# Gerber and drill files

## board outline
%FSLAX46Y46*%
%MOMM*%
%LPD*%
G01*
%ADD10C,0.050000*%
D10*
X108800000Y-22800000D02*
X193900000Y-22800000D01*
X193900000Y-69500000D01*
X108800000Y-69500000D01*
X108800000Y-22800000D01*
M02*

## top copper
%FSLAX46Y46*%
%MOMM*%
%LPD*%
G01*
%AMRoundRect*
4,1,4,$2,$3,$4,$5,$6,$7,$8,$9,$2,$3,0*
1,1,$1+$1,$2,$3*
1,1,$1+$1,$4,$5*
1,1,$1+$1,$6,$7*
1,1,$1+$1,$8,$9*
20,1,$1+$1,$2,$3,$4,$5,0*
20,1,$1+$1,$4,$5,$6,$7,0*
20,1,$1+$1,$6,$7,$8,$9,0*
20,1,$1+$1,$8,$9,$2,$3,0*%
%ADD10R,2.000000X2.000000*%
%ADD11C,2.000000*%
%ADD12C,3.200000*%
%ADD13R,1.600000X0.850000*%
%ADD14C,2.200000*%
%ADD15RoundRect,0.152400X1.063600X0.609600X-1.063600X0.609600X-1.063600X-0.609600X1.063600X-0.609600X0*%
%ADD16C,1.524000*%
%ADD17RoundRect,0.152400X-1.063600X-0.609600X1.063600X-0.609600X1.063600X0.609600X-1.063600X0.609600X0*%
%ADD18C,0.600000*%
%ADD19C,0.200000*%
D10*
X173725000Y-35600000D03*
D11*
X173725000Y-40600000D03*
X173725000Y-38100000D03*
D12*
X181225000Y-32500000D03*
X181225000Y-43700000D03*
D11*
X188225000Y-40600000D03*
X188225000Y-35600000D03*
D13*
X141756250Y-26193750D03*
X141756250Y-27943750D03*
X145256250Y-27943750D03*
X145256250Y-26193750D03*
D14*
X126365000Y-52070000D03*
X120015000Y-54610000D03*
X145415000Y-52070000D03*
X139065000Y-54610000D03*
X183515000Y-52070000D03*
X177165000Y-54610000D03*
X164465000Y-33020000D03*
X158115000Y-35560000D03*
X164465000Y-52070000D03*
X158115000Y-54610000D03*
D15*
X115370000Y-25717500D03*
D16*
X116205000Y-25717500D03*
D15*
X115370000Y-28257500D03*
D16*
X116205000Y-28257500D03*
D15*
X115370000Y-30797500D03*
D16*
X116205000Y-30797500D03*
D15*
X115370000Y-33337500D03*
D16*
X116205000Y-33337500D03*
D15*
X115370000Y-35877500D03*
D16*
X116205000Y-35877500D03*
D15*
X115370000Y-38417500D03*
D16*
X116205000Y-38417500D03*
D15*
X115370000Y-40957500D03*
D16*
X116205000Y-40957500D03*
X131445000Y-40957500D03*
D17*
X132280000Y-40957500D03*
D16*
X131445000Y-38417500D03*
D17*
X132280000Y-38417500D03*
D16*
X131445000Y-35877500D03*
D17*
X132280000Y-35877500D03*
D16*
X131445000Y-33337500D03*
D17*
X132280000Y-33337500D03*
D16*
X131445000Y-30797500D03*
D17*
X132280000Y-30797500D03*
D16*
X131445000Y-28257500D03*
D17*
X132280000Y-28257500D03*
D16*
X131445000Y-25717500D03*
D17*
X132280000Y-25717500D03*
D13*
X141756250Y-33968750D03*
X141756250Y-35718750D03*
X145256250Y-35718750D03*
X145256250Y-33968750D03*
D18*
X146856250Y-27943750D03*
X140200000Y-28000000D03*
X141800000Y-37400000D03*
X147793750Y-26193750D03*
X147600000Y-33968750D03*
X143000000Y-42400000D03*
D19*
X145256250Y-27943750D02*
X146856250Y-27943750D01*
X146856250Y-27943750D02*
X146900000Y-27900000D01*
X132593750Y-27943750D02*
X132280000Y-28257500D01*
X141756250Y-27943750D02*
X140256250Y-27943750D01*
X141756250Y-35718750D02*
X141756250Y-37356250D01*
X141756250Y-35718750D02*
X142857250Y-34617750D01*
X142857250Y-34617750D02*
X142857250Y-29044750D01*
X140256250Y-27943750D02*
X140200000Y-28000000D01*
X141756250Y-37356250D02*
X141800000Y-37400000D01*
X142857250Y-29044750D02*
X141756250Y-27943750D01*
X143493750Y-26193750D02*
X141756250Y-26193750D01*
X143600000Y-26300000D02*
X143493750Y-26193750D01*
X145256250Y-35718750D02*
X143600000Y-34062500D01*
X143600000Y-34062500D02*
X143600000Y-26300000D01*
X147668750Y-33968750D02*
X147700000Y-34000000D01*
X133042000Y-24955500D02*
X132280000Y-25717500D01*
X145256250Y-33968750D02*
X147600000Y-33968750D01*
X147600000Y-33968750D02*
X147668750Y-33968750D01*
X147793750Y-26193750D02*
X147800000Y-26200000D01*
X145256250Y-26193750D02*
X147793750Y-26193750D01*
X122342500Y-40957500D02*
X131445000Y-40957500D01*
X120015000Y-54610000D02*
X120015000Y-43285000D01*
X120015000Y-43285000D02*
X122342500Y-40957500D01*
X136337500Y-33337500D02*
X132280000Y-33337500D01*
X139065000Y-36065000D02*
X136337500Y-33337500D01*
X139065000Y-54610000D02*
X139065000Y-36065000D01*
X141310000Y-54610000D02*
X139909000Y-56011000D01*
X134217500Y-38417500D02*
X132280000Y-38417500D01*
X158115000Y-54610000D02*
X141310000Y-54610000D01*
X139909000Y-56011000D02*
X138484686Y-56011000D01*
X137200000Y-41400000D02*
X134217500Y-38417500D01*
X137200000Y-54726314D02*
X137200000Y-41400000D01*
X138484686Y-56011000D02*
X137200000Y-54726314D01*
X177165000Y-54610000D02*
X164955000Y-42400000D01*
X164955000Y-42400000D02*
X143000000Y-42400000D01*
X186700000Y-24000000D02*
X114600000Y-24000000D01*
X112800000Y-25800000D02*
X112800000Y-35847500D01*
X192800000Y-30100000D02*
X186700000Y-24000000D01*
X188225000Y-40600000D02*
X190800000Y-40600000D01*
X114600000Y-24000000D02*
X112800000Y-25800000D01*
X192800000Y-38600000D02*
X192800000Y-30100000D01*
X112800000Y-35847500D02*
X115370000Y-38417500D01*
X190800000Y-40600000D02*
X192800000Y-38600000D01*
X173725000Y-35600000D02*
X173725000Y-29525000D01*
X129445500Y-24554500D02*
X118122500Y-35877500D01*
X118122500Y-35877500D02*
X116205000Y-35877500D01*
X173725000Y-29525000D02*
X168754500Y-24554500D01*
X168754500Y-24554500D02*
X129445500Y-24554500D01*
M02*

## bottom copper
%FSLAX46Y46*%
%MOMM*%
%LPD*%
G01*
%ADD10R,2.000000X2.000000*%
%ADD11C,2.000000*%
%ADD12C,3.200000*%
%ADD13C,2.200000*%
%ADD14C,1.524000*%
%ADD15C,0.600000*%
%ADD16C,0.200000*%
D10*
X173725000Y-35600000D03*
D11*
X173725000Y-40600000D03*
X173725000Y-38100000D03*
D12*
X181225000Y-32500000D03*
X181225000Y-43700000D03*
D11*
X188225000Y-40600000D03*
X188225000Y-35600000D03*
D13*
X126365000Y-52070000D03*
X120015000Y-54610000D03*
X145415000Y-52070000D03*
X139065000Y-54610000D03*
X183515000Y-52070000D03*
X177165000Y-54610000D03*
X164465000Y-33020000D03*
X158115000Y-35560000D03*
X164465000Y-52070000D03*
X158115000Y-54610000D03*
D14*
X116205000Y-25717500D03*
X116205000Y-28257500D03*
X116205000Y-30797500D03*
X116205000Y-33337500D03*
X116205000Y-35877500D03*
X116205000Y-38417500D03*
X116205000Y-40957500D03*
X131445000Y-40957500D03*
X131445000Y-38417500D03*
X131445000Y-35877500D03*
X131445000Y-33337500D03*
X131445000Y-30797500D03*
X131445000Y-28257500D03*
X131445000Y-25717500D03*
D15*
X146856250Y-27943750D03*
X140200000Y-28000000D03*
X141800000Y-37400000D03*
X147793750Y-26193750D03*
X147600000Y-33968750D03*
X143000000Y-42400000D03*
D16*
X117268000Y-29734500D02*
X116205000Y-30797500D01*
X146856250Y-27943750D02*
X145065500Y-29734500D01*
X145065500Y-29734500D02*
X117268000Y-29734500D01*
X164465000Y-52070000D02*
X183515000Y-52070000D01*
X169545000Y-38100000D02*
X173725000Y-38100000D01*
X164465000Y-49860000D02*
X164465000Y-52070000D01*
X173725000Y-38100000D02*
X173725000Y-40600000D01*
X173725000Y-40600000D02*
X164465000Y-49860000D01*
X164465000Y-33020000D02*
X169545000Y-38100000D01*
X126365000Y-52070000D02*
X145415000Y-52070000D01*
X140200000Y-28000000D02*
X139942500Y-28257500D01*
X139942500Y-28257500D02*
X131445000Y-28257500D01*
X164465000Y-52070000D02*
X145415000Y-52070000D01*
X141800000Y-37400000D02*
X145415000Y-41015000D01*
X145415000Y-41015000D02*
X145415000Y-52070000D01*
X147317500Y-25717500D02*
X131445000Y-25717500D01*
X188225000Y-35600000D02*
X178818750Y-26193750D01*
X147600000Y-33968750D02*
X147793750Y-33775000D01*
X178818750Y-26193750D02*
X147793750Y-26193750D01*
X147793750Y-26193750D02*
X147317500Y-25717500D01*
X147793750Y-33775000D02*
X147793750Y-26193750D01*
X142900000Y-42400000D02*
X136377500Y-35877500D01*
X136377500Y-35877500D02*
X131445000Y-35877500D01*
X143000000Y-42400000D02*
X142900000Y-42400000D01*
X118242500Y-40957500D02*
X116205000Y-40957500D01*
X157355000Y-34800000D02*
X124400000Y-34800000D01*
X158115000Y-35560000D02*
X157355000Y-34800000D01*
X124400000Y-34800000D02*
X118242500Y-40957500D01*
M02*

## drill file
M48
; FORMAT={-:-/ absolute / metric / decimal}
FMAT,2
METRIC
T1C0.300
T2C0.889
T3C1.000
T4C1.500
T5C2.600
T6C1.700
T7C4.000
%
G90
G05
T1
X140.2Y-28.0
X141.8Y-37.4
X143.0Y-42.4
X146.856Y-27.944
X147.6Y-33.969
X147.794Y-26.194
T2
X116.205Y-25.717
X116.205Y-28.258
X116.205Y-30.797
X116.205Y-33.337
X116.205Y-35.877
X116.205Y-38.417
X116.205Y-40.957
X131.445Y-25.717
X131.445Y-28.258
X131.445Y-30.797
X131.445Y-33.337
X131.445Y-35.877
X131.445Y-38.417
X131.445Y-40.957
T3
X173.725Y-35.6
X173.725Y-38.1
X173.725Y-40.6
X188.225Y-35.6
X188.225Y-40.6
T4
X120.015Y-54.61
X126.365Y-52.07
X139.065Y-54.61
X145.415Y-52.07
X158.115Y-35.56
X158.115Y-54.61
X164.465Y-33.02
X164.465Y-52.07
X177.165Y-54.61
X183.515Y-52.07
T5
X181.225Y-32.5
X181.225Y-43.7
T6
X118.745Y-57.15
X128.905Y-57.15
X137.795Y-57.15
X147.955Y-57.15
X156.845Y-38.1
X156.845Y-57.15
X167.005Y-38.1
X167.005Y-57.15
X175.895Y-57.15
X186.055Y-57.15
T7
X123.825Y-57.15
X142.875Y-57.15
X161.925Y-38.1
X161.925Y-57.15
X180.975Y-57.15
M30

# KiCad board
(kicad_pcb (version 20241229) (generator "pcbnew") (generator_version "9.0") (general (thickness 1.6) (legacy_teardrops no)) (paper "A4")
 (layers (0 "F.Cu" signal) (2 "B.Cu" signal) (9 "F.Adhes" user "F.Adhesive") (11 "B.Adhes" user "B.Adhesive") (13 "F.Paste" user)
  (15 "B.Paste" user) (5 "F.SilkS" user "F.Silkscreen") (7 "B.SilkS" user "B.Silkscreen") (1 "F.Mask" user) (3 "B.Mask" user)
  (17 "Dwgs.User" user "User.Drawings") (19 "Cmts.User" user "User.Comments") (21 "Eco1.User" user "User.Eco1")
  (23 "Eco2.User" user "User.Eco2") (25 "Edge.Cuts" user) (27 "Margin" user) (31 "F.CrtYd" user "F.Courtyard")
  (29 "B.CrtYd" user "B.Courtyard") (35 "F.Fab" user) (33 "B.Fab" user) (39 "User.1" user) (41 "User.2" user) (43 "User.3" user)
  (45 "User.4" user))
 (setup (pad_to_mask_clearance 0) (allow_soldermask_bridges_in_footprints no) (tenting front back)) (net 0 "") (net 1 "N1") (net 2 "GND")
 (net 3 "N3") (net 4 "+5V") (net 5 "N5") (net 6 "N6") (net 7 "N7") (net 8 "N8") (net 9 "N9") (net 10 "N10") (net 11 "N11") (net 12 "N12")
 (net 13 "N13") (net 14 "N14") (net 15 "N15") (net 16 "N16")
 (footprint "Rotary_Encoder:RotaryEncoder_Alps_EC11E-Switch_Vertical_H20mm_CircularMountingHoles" (layer "F.Cu") (at 173.725 35.6)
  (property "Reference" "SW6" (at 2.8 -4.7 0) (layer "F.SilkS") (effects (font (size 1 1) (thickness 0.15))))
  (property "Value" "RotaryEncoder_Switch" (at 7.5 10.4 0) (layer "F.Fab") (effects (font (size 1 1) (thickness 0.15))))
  (pad "A" thru_hole rect (at 0 0) (size 2 2) (drill 1) (layers "*.Cu" "*.Mask") (remove_unused_layers no) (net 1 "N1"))
  (pad "B" thru_hole circle (at 0 5) (size 2 2) (drill 1) (layers "*.Cu" "*.Mask") (remove_unused_layers no) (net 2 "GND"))
  (pad "C" thru_hole circle (at 0 2.5) (size 2 2) (drill 1) (layers "*.Cu" "*.Mask") (remove_unused_layers no) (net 2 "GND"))
  (pad "MP" thru_hole circle (at 7.5 -3.1) (size 3.2 3.2) (drill 2.6) (layers "*.Cu" "*.Mask") (remove_unused_layers no))
  (pad "MP" thru_hole circle (at 7.5 8.1) (size 3.2 3.2) (drill 2.6) (layers "*.Cu" "*.Mask") (remove_unused_layers no))
  (pad "S1" thru_hole circle (at 14.5 5) (size 2 2) (drill 1) (layers "*.Cu" "*.Mask") (remove_unused_layers no) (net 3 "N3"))
  (pad "S2" thru_hole circle (at 14.5 0) (size 2 2) (drill 1) (layers "*.Cu" "*.Mask") (remove_unused_layers no) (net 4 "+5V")))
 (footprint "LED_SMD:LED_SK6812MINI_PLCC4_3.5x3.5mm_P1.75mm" (layer "F.Cu") (at 143.50625 27.06875)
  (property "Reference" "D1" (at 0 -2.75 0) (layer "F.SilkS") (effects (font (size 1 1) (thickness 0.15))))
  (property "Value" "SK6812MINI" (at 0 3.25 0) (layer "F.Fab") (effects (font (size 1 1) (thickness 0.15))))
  (pad "1" smd rect (at -1.75 -0.875) (size 1.6 0.85) (layers "F.Cu" "F.Mask" "F.Paste") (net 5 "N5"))
  (pad "2" smd rect (at -1.75 0.875) (size 1.6 0.85) (layers "F.Cu" "F.Mask" "F.Paste") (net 2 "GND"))
  (pad "3" smd rect (at 1.75 0.875) (size 1.6 0.85) (layers "F.Cu" "F.Mask" "F.Paste") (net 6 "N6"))
  (pad "4" smd rect (at 1.75 -0.875) (size 1.6 0.85) (layers "F.Cu" "F.Mask" "F.Paste") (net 4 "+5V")))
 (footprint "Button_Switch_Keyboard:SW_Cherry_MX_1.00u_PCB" (layer "F.Cu") (at 126.365 52.07)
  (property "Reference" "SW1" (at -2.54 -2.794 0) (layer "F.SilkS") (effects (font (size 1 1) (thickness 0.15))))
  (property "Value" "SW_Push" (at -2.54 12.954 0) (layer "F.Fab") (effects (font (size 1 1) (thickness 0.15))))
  (pad "" np_thru_hole circle (at -7.62 5.08) (size 1.7 1.7) (drill 1.7) (layers "*.Cu" "*.Mask"))
  (pad "" np_thru_hole circle (at -2.54 5.08) (size 4 4) (drill 4) (layers "*.Cu" "*.Mask"))
  (pad "" np_thru_hole circle (at 2.54 5.08) (size 1.7 1.7) (drill 1.7) (layers "*.Cu" "*.Mask"))
  (pad "1" thru_hole circle (at 0 0) (size 2.2 2.2) (drill 1.5) (layers "*.Cu" "*.Mask") (remove_unused_layers no) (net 2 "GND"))
  (pad "2" thru_hole circle (at -6.35 2.54) (size 2.2 2.2) (drill 1.5) (layers "*.Cu" "*.Mask") (remove_unused_layers no) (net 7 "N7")))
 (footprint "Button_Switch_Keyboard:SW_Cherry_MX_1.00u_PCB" (layer "F.Cu") (at 145.415 52.07)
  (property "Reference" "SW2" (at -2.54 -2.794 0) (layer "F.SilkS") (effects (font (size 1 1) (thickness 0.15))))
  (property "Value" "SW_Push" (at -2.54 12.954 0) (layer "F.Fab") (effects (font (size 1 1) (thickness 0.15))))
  (pad "" np_thru_hole circle (at -7.62 5.08) (size 1.7 1.7) (drill 1.7) (layers "*.Cu" "*.Mask"))
  (pad "" np_thru_hole circle (at -2.54 5.08) (size 4 4) (drill 4) (layers "*.Cu" "*.Mask"))
  (pad "" np_thru_hole circle (at 2.54 5.08) (size 1.7 1.7) (drill 1.7) (layers "*.Cu" "*.Mask"))
  (pad "1" thru_hole circle (at 0 0) (size 2.2 2.2) (drill 1.5) (layers "*.Cu" "*.Mask") (remove_unused_layers no) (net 2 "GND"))
  (pad "2" thru_hole circle (at -6.35 2.54) (size 2.2 2.2) (drill 1.5) (layers "*.Cu" "*.Mask") (remove_unused_layers no) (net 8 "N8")))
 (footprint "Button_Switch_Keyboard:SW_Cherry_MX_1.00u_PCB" (layer "F.Cu") (at 183.515 52.07)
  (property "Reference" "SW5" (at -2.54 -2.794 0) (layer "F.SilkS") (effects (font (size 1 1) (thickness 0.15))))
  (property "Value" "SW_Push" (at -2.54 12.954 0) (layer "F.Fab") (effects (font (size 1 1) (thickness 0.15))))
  (pad "" np_thru_hole circle (at -7.62 5.08) (size 1.7 1.7) (drill 1.7) (layers "*.Cu" "*.Mask"))
  (pad "" np_thru_hole circle (at -2.54 5.08) (size 4 4) (drill 4) (layers "*.Cu" "*.Mask"))
  (pad "" np_thru_hole circle (at 2.54 5.08) (size 1.7 1.7) (drill 1.7) (layers "*.Cu" "*.Mask"))
  (pad "1" thru_hole circle (at 0 0) (size 2.2 2.2) (drill 1.5) (layers "*.Cu" "*.Mask") (remove_unused_layers no) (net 2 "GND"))
  (pad "2" thru_hole circle (at -6.35 2.54) (size 2.2 2.2) (drill 1.5) (layers "*.Cu" "*.Mask") (remove_unused_layers no) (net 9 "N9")))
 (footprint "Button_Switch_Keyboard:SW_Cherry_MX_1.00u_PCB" (layer "F.Cu") (at 164.465 33.02)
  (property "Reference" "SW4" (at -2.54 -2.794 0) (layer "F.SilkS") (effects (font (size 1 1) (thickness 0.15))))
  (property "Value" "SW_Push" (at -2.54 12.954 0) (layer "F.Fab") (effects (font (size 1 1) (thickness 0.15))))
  (pad "" np_thru_hole circle (at -7.62 5.08) (size 1.7 1.7) (drill 1.7) (layers "*.Cu" "*.Mask"))
  (pad "" np_thru_hole circle (at -2.54 5.08) (size 4 4) (drill 4) (layers "*.Cu" "*.Mask"))
  (pad "" np_thru_hole circle (at 2.54 5.08) (size 1.7 1.7) (drill 1.7) (layers "*.Cu" "*.Mask"))
  (pad "1" thru_hole circle (at 0 0) (size 2.2 2.2) (drill 1.5) (layers "*.Cu" "*.Mask") (remove_unused_layers no) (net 2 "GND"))
  (pad "2" thru_hole circle (at -6.35 2.54) (size 2.2 2.2) (drill 1.5) (layers "*.Cu" "*.Mask") (remove_unused_layers no) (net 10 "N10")))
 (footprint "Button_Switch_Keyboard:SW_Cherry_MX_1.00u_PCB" (layer "F.Cu") (at 164.465 52.07)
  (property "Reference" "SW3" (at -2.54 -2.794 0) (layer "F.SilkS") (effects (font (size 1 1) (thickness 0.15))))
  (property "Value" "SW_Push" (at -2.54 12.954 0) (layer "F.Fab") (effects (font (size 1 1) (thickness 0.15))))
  (pad "" np_thru_hole circle (at -7.62 5.08) (size 1.7 1.7) (drill 1.7) (layers "*.Cu" "*.Mask"))
  (pad "" np_thru_hole circle (at -2.54 5.08) (size 4 4) (drill 4) (layers "*.Cu" "*.Mask"))
  (pad "" np_thru_hole circle (at 2.54 5.08) (size 1.7 1.7) (drill 1.7) (layers "*.Cu" "*.Mask"))
  (pad "1" thru_hole circle (at 0 0) (size 2.2 2.2) (drill 1.5) (layers "*.Cu" "*.Mask") (remove_unused_layers no) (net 2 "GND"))
  (pad "2" thru_hole circle (at -6.35 2.54) (size 2.2 2.2) (drill 1.5) (layers "*.Cu" "*.Mask") (remove_unused_layers no) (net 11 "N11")))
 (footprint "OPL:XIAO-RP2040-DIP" (layer "F.Cu") (at 123.825 33.3375)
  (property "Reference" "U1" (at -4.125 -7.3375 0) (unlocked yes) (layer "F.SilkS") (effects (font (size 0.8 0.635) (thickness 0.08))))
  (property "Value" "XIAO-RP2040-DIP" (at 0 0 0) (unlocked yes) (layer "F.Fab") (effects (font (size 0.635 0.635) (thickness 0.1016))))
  (pad "1" smd roundrect (at -8.455 -7.62 180) (size 2.432 1.524) (layers "F.Cu" "F.Mask") (roundrect_rratio 0.1) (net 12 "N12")
   (thermal_bridge_angle 45))
  (pad "1" thru_hole circle (at -7.62 -7.62 180) (size 1.524 1.524) (drill 0.889) (layers "*.Cu" "*.Mask") (remove_unused_layers no)
   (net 12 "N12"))
  (pad "2" smd roundrect (at -8.455 -5.08 180) (size 2.432 1.524) (layers "F.Cu" "F.Mask") (roundrect_rratio 0.1) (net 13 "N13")
   (thermal_bridge_angle 45))
  (pad "2" thru_hole circle (at -7.62 -5.08 180) (size 1.524 1.524) (drill 0.889) (layers "*.Cu" "*.Mask") (remove_unused_layers no)
   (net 13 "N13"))
  (pad "3" smd roundrect (at -8.455 -2.54 180) (size 2.432 1.524) (layers "F.Cu" "F.Mask") (roundrect_rratio 0.1) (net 6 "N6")
   (thermal_bridge_angle 45))
  (pad "3" thru_hole circle (at -7.62 -2.54 180) (size 1.524 1.524) (drill 0.889) (layers "*.Cu" "*.Mask") (remove_unused_layers no)
   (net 6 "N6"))
  (pad "4" smd roundrect (at -8.455 0 180) (size 2.432 1.524) (layers "F.Cu" "F.Mask") (roundrect_rratio 0.1) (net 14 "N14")
   (thermal_bridge_angle 45))
  (pad "4" thru_hole circle (at -7.62 0 180) (size 1.524 1.524) (drill 0.889) (layers "*.Cu" "*.Mask") (remove_unused_layers no)
   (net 14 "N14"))
  (pad "5" smd roundrect (at -8.455 2.54 180) (size 2.432 1.524) (layers "F.Cu" "F.Mask") (roundrect_rratio 0.1) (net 1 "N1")
   (thermal_bridge_angle 45))
  (pad "5" thru_hole circle (at -7.62 2.54 180) (size 1.524 1.524) (drill 0.889) (layers "*.Cu" "*.Mask") (remove_unused_layers no)
   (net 1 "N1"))
  (pad "6" smd roundrect (at -8.455 5.08 180) (size 2.432 1.524) (layers "F.Cu" "F.Mask") (roundrect_rratio 0.1) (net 3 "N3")
   (thermal_bridge_angle 45))
  (pad "6" thru_hole circle (at -7.62 5.08 180) (size 1.524 1.524) (drill 0.889) (layers "*.Cu" "*.Mask") (remove_unused_layers no)
   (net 3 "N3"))
  (pad "7" smd roundrect (at -8.455 7.62 180) (size 2.432 1.524) (layers "F.Cu" "F.Mask") (roundrect_rratio 0.1) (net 10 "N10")
   (thermal_bridge_angle 45))
  (pad "7" thru_hole circle (at -7.62 7.62 180) (size 1.524 1.524) (drill 0.889) (layers "*.Cu" "*.Mask") (remove_unused_layers no)
   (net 10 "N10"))
  (pad "8" thru_hole circle (at 7.62 7.62) (size 1.524 1.524) (drill 0.889) (layers "*.Cu" "*.Mask") (remove_unused_layers no) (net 7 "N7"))
  (pad "8" smd roundrect (at 8.455 7.62) (size 2.432 1.524) (layers "F.Cu" "F.Mask") (roundrect_rratio 0.1) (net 7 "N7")
   (thermal_bridge_angle 45))
  (pad "9" thru_hole circle (at 7.62 5.08) (size 1.524 1.524) (drill 0.889) (layers "*.Cu" "*.Mask") (remove_unused_layers no)
   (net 11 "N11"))
  (pad "9" smd roundrect (at 8.455 5.08) (size 2.432 1.524) (layers "F.Cu" "F.Mask") (roundrect_rratio 0.1) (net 11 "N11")
   (thermal_bridge_angle 45))
  (pad "10" thru_hole circle (at 7.62 2.54) (size 1.524 1.524) (drill 0.889) (layers "*.Cu" "*.Mask") (remove_unused_layers no) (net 9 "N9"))
  (pad "10" smd roundrect (at 8.455 2.54) (size 2.432 1.524) (layers "F.Cu" "F.Mask") (roundrect_rratio 0.1) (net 9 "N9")
   (thermal_bridge_angle 45))
  (pad "11" thru_hole circle (at 7.62 0) (size 1.524 1.524) (drill 0.889) (layers "*.Cu" "*.Mask") (remove_unused_layers no) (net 8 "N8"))
  (pad "11" smd roundrect (at 8.455 0) (size 2.432 1.524) (layers "F.Cu" "F.Mask") (roundrect_rratio 0.1) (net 8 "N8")
   (thermal_bridge_angle 45))
  (pad "12" thru_hole circle (at 7.62 -2.54) (size 1.524 1.524) (drill 0.889) (layers "*.Cu" "*.Mask") (remove_unused_layers no)
   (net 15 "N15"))
  (pad "12" smd roundrect (at 8.455 -2.54) (size 2.432 1.524) (layers "F.Cu" "F.Mask") (roundrect_rratio 0.1) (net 15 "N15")
   (thermal_bridge_angle 45))
  (pad "13" thru_hole circle (at 7.62 -5.08) (size 1.524 1.524) (drill 0.889) (layers "*.Cu" "*.Mask") (remove_unused_layers no)
   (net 2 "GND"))
  (pad "13" smd roundrect (at 8.455 -5.08) (size 2.432 1.524) (layers "F.Cu" "F.Mask") (roundrect_rratio 0.1) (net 2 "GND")
   (thermal_bridge_angle 45))
  (pad "14" thru_hole circle (at 7.62 -7.62) (size 1.524 1.524) (drill 0.889) (layers "*.Cu" "*.Mask") (remove_unused_layers no)
   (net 4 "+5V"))
  (pad "14" smd roundrect (at 8.455 -7.62) (size 2.432 1.524) (layers "F.Cu" "F.Mask") (roundrect_rratio 0.1) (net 4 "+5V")
   (thermal_bridge_angle 45)))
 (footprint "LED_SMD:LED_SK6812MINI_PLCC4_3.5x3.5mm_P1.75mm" (layer "F.Cu") (at 143.50625 34.84375)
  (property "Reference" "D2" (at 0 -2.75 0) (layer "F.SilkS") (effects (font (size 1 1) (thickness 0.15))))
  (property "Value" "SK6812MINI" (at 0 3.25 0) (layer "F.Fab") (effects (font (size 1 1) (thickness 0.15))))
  (pad "1" smd rect (at -1.75 -0.875) (size 1.6 0.85) (layers "F.Cu" "F.Mask" "F.Paste") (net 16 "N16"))
  (pad "2" smd rect (at -1.75 0.875) (size 1.6 0.85) (layers "F.Cu" "F.Mask" "F.Paste") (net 2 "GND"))
  (pad "3" smd rect (at 1.75 0.875) (size 1.6 0.85) (layers "F.Cu" "F.Mask" "F.Paste") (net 5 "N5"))
  (pad "4" smd rect (at 1.75 -0.875) (size 1.6 0.85) (layers "F.Cu" "F.Mask" "F.Paste") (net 4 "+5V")))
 (gr_rect (start 108.8 22.8) (end 193.9 69.5) (stroke (width 0.05) (type default)) (fill no) (layer "Edge.Cuts"))
 (segment (start 145.25625 27.94375) (end 146.85625 27.94375) (width 0.2) (layer "F.Cu") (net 6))
 (segment (start 146.85625 27.94375) (end 146.9 27.9) (width 0.2) (layer "F.Cu") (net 6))
 (via (at 146.85625 27.94375) (size 0.6) (drill 0.3) (layers "F.Cu" "B.Cu") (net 6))
 (segment (start 117.268 29.7345) (end 116.205 30.7975) (width 0.2) (layer "B.Cu") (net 6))
 (segment (start 146.85625 27.94375) (end 145.0655 29.7345) (width 0.2) (layer "B.Cu") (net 6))
 (segment (start 145.0655 29.7345) (end 117.268 29.7345) (width 0.2) (layer "B.Cu") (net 6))
 (segment (start 132.59375 27.94375) (end 132.28 28.2575) (width 0.2) (layer "F.Cu") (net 2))
 (segment (start 141.75625 27.94375) (end 140.25625 27.94375) (width 0.2) (layer "F.Cu") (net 2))
 (segment (start 141.75625 35.71875) (end 141.75625 37.35625) (width 0.2) (layer "F.Cu") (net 2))
 (segment (start 141.75625 35.71875) (end 142.85725 34.61775) (width 0.2) (layer "F.Cu") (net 2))
 (segment (start 142.85725 34.61775) (end 142.85725 29.04475) (width 0.2) (layer "F.Cu") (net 2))
 (segment (start 140.25625 27.94375) (end 140.2 28) (width 0.2) (layer "F.Cu") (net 2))
 (segment (start 141.75625 37.35625) (end 141.8 37.4) (width 0.2) (layer "F.Cu") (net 2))
 (segment (start 142.85725 29.04475) (end 141.75625 27.94375) (width 0.2) (layer "F.Cu") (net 2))
 (via (at 140.2 28) (size 0.6) (drill 0.3) (layers "F.Cu" "B.Cu") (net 2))
 (via (at 141.8 37.4) (size 0.6) (drill 0.3) (layers "F.Cu" "B.Cu") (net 2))
 (segment (start 164.465 52.07) (end 183.515 52.07) (width 0.2) (layer "B.Cu") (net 2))
 (segment (start 169.545 38.1) (end 173.725 38.1) (width 0.2) (layer "B.Cu") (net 2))
 (segment (start 164.465 49.86) (end 164.465 52.07) (width 0.2) (layer "B.Cu") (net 2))
 (segment (start 173.725 38.1) (end 173.725 40.6) (width 0.2) (layer "B.Cu") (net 2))
 (segment (start 173.725 40.6) (end 164.465 49.86) (width 0.2) (layer "B.Cu") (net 2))
 (segment (start 164.465 33.02) (end 169.545 38.1) (width 0.2) (layer "B.Cu") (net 2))
 (segment (start 126.365 52.07) (end 145.415 52.07) (width 0.2) (layer "B.Cu") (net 2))
 (segment (start 140.2 28) (end 139.9425 28.2575) (width 0.2) (layer "B.Cu") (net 2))
 (segment (start 139.9425 28.2575) (end 131.445 28.2575) (width 0.2) (layer "B.Cu") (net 2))
 (segment (start 164.465 52.07) (end 145.415 52.07) (width 0.2) (layer "B.Cu") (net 2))
 (segment (start 141.8 37.4) (end 145.415 41.015) (width 0.2) (layer "B.Cu") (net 2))
 (segment (start 145.415 41.015) (end 145.415 52.07) (width 0.2) (layer "B.Cu") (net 2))
 (segment (start 143.49375 26.19375) (end 141.75625 26.19375) (width 0.2) (layer "F.Cu") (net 5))
 (segment (start 143.6 26.3) (end 143.49375 26.19375) (width 0.2) (layer "F.Cu") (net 5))
 (segment (start 145.25625 35.71875) (end 143.6 34.0625) (width 0.2) (layer "F.Cu") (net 5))
 (segment (start 143.6 34.0625) (end 143.6 26.3) (width 0.2) (layer "F.Cu") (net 5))
 (segment (start 147.66875 33.96875) (end 147.7 34) (width 0.2) (layer "F.Cu") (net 4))
 (segment (start 133.042 24.9555) (end 132.28 25.7175) (width 0.2) (layer "F.Cu") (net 4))
 (segment (start 145.25625 33.96875) (end 147.6 33.96875) (width 0.2) (layer "F.Cu") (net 4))
 (segment (start 147.6 33.96875) (end 147.66875 33.96875) (width 0.2) (layer "F.Cu") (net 4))
 (segment (start 147.79375 26.19375) (end 147.8 26.2) (width 0.2) (layer "F.Cu") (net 4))
 (segment (start 145.25625 26.19375) (end 147.79375 26.19375) (width 0.2) (layer "F.Cu") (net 4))
 (via (at 147.79375 26.19375) (size 0.6) (drill 0.3) (layers "F.Cu" "B.Cu") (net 4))
 (via (at 147.6 33.96875) (size 0.6) (drill 0.3) (layers "F.Cu" "B.Cu") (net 4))
 (segment (start 147.3175 25.7175) (end 131.445 25.7175) (width 0.2) (layer "B.Cu") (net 4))
 (segment (start 188.225 35.6) (end 178.81875 26.19375) (width 0.2) (layer "B.Cu") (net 4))
 (segment (start 147.6 33.96875) (end 147.79375 33.775) (width 0.2) (layer "B.Cu") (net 4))
 (segment (start 178.81875 26.19375) (end 147.79375 26.19375) (width 0.2) (layer "B.Cu") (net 4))
 (segment (start 147.79375 26.19375) (end 147.3175 25.7175) (width 0.2) (layer "B.Cu") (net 4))
 (segment (start 147.79375 33.775) (end 147.79375 26.19375) (width 0.2) (layer "B.Cu") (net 4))
 (segment (start 122.3425 40.9575) (end 131.445 40.9575) (width 0.2) (layer "F.Cu") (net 7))
 (segment (start 120.015 54.61) (end 120.015 43.285) (width 0.2) (layer "F.Cu") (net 7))
 (segment (start 120.015 43.285) (end 122.3425 40.9575) (width 0.2) (layer "F.Cu") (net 7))
 (segment (start 136.3375 33.3375) (end 132.28 33.3375) (width 0.2) (layer "F.Cu") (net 8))
 (segment (start 139.065 36.065) (end 136.3375 33.3375) (width 0.2) (layer "F.Cu") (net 8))
 (segment (start 139.065 54.61) (end 139.065 36.065) (width 0.2) (layer "F.Cu") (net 8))
 (segment (start 141.31 54.61) (end 139.909 56.011) (width 0.2) (layer "F.Cu") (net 11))
 (segment (start 134.2175 38.4175) (end 132.28 38.4175) (width 0.2) (layer "F.Cu") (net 11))
 (segment (start 158.115 54.61) (end 141.31 54.61) (width 0.2) (layer "F.Cu") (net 11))
 (segment (start 139.909 56.011) (end 138.484686 56.011) (width 0.2) (layer "F.Cu") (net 11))
 (segment (start 137.2 41.4) (end 134.2175 38.4175) (width 0.2) (layer "F.Cu") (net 11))
 (segment (start 137.2 54.726314) (end 137.2 41.4) (width 0.2) (layer "F.Cu") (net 11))
 (segment (start 138.484686 56.011) (end 137.2 54.726314) (width 0.2) (layer "F.Cu") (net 11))
 (segment (start 177.165 54.61) (end 164.955 42.4) (width 0.2) (layer "F.Cu") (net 9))
 (segment (start 164.955 42.4) (end 143 42.4) (width 0.2) (layer "F.Cu") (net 9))
 (via (at 143 42.4) (size 0.6) (drill 0.3) (layers "F.Cu" "B.Cu") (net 9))
 (segment (start 142.9 42.4) (end 136.3775 35.8775) (width 0.2) (layer "B.Cu") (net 9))
 (segment (start 136.3775 35.8775) (end 131.445 35.8775) (width 0.2) (layer "B.Cu") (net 9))
 (segment (start 143 42.4) (end 142.9 42.4) (width 0.2) (layer "B.Cu") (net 9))
 (segment (start 118.2425 40.9575) (end 116.205 40.9575) (width 0.2) (layer "B.Cu") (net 10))
 (segment (start 157.355 34.8) (end 124.4 34.8) (width 0.2) (layer "B.Cu") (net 10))
 (segment (start 158.115 35.56) (end 157.355 34.8) (width 0.2) (layer "B.Cu") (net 10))
 (segment (start 124.4 34.8) (end 118.2425 40.9575) (width 0.2) (layer "B.Cu") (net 10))
 (segment (start 186.7 24) (end 114.6 24) (width 0.2) (layer "F.Cu") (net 3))
 (segment (start 112.8 25.8) (end 112.8 35.8475) (width 0.2) (layer "F.Cu") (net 3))
 (segment (start 192.8 30.1) (end 186.7 24) (width 0.2) (layer "F.Cu") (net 3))
 (segment (start 188.225 40.6) (end 190.8 40.6) (width 0.2) (layer "F.Cu") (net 3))
 (segment (start 114.6 24) (end 112.8 25.8) (width 0.2) (layer "F.Cu") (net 3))
 (segment (start 192.8 38.6) (end 192.8 30.1) (width 0.2) (layer "F.Cu") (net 3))
 (segment (start 112.8 35.8475) (end 115.37 38.4175) (width 0.2) (layer "F.Cu") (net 3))
 (segment (start 190.8 40.6) (end 192.8 38.6) (width 0.2) (layer "F.Cu") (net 3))
 (segment (start 173.725 35.6) (end 173.725 29.525) (width 0.2) (layer "F.Cu") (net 1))
 (segment (start 129.4455 24.5545) (end 118.1225 35.8775) (width 0.2) (layer "F.Cu") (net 1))
 (segment (start 118.1225 35.8775) (end 116.205 35.8775) (width 0.2) (layer "F.Cu") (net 1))
 (segment (start 173.725 29.525) (end 168.7545 24.5545) (width 0.2) (layer "F.Cu") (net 1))
 (segment (start 168.7545 24.5545) (end 129.4455 24.5545) (width 0.2) (layer "F.Cu") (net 1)))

